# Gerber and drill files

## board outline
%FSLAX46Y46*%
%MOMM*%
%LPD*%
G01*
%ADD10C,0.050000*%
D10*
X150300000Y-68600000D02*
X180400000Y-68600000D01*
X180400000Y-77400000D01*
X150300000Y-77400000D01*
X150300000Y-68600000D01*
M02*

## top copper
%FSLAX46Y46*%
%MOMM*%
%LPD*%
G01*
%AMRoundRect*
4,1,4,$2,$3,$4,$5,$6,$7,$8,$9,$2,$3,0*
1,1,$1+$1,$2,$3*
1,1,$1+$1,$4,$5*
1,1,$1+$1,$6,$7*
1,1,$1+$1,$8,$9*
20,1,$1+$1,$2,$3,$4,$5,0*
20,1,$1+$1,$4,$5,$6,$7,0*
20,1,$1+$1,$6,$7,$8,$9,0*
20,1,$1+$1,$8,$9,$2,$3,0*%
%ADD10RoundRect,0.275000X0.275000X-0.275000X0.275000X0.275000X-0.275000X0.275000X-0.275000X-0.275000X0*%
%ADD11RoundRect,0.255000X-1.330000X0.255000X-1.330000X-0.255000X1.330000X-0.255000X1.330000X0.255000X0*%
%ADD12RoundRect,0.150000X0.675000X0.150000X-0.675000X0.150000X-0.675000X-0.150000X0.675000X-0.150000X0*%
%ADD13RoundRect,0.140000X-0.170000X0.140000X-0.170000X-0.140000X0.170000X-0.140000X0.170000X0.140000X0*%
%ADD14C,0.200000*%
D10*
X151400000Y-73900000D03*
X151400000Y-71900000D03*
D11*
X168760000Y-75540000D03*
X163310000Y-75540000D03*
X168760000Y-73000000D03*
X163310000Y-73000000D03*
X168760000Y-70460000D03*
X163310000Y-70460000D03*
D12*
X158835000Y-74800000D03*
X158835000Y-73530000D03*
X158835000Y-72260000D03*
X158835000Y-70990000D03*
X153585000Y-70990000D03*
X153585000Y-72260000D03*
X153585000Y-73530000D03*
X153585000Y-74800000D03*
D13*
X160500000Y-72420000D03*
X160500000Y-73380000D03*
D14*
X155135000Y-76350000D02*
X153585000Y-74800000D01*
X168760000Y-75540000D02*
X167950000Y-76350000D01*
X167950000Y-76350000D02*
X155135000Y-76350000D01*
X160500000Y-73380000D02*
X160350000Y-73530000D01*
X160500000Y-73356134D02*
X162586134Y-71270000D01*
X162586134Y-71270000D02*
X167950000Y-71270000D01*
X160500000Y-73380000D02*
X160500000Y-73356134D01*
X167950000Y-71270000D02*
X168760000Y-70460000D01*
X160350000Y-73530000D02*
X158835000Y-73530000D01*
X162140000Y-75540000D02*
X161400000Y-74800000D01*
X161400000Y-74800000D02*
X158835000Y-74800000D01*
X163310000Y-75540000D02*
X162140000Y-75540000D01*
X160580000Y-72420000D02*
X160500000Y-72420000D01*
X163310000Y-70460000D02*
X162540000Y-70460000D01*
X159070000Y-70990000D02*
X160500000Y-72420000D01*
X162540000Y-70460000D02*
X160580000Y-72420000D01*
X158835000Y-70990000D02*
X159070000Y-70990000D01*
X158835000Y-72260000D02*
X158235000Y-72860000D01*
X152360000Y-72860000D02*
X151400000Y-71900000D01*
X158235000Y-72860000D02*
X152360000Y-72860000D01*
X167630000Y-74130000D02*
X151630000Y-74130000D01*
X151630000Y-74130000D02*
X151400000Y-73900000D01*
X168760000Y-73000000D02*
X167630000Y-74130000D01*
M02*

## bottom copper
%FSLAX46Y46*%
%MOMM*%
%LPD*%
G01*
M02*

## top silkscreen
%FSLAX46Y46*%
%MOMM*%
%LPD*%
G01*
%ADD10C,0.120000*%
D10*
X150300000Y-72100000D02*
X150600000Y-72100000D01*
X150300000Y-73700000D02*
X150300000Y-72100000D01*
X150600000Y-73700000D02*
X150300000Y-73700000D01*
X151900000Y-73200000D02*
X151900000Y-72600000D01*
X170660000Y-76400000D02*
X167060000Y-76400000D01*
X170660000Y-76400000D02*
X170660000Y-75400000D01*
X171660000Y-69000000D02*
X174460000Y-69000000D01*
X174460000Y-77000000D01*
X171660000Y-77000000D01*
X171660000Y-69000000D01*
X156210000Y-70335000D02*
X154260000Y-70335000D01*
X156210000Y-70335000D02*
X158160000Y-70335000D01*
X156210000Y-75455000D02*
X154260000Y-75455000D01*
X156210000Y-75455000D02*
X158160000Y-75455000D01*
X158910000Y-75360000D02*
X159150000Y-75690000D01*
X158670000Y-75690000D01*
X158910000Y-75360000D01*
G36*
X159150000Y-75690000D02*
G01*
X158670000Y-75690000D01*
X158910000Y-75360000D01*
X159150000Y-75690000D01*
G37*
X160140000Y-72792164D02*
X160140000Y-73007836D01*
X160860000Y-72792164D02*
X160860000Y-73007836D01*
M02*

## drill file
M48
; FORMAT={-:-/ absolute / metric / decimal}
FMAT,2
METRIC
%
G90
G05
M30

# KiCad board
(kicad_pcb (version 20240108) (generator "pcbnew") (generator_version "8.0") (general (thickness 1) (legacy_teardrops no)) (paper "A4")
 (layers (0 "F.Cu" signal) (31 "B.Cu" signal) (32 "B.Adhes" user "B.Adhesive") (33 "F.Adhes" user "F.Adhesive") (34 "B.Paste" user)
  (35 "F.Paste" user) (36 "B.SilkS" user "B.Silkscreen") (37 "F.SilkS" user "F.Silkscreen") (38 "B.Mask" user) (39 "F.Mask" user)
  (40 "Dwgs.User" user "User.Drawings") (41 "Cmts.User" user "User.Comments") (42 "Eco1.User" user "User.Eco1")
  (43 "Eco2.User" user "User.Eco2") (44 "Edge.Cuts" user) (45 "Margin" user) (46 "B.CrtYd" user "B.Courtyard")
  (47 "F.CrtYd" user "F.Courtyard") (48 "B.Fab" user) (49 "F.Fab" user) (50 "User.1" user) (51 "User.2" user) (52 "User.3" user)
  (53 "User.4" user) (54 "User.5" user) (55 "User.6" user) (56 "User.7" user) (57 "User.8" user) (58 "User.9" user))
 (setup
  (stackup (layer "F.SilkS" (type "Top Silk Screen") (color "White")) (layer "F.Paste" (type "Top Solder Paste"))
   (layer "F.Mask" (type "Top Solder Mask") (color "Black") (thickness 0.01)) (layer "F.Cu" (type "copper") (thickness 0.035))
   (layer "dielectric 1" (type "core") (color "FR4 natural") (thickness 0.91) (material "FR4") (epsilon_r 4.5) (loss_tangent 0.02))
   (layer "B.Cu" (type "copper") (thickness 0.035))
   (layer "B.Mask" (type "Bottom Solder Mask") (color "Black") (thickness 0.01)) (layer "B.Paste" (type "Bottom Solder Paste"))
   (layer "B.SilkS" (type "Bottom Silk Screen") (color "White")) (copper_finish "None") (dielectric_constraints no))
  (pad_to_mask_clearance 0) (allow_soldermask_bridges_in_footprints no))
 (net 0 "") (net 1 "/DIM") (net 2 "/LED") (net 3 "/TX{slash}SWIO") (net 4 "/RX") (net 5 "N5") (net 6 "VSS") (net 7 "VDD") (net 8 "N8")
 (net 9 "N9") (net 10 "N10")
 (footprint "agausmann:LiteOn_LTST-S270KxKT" (layer "F.Cu") (at 151.4 72.9 90)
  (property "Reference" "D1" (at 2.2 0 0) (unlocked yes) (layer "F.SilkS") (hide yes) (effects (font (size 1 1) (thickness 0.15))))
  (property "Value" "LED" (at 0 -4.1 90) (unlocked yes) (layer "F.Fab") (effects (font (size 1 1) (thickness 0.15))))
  (fp_line (start 0.8 -1.1) (end 0.8 -0.8) (stroke (width 0.12) (type default)) (layer "F.SilkS"))
  (fp_line (start -0.8 -1.1) (end 0.8 -1.1) (stroke (width 0.12) (type default)) (layer "F.SilkS"))
  (fp_line (start -0.8 -0.8) (end -0.8 -1.1) (stroke (width 0.12) (type default)) (layer "F.SilkS"))
  (fp_line (start -0.3 0.5) (end 0.3 0.5) (stroke (width 0.12) (type default)) (layer "F.SilkS"))
  (pad "1" smd roundrect (at -1 0 90) (size 1.1 1.1) (layers "F.Cu" "F.Paste" "F.Mask") (roundrect_rratio 0.25) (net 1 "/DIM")
   (thermal_bridge_angle 45))
  (pad "2" smd roundrect (at 1 0 90) (size 1.1 1.1) (layers "F.Cu" "F.Paste" "F.Mask") (roundrect_rratio 0.25) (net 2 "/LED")
   (thermal_bridge_angle 45)))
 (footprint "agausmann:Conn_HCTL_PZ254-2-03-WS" (layer "F.Cu") (at 173.06 73 90)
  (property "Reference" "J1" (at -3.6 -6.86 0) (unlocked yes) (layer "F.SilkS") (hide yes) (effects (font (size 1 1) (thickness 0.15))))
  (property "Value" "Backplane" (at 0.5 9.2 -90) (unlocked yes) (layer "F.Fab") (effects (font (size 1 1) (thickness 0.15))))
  (fp_line (start -3.4 -2.4) (end -3.4 -6) (stroke (width 0.12) (type default)) (layer "F.SilkS"))
  (fp_line (start -3.4 -2.4) (end -2.4 -2.4) (stroke (width 0.12) (type default)) (layer "F.SilkS"))
  (fp_rect (start -4 -1.4) (end 4 1.4) (stroke (width 0.12) (type default)) (fill none) (layer "F.SilkS"))
  (pad "1" smd roundrect (at -2.54 -4.3 270) (size 1.02 3.17) (layers "F.Cu" "F.Paste" "F.Mask") (roundrect_rratio 0.25)
   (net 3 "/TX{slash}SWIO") (thermal_bridge_angle 45))
  (pad "2" smd roundrect (at -2.54 -9.75 270) (size 1.02 3.17) (layers "F.Cu" "F.Paste" "F.Mask") (roundrect_rratio 0.25) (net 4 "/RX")
   (thermal_bridge_angle 45))
  (pad "3" smd roundrect (at 0 -4.3 270) (size 1.02 3.17) (layers "F.Cu" "F.Paste" "F.Mask") (roundrect_rratio 0.25) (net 1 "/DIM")
   (thermal_bridge_angle 45))
  (pad "4" smd roundrect (at 0 -9.75 270) (size 1.02 3.17) (layers "F.Cu" "F.Paste" "F.Mask") (roundrect_rratio 0.25) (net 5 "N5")
   (thermal_bridge_angle 45))
  (pad "5" smd roundrect (at 2.54 -4.3 270) (size 1.02 3.17) (layers "F.Cu" "F.Paste" "F.Mask") (roundrect_rratio 0.25) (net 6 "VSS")
   (thermal_bridge_angle 45))
  (pad "6" smd roundrect (at 2.54 -9.75 270) (size 1.02 3.17) (layers "F.Cu" "F.Paste" "F.Mask") (roundrect_rratio 0.25) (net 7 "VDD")
   (thermal_bridge_angle 45)))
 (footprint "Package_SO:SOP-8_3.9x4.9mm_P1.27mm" (layer "F.Cu") (at 156.21 72.895 180)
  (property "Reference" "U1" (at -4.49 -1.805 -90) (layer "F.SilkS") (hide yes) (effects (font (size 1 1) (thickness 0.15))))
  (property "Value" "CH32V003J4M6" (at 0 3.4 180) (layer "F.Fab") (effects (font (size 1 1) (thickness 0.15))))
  (fp_line (start 0 2.56) (end 1.95 2.56) (stroke (width 0.12) (type solid)) (layer "F.SilkS"))
  (fp_line (start 0 2.56) (end -1.95 2.56) (stroke (width 0.12) (type solid)) (layer "F.SilkS"))
  (fp_line (start 0 -2.56) (end 1.95 -2.56) (stroke (width 0.12) (type solid)) (layer "F.SilkS"))
  (fp_line (start 0 -2.56) (end -1.95 -2.56) (stroke (width 0.12) (type solid)) (layer "F.SilkS"))
  (fp_poly
   (pts (xy -2.7 -2.465) (xy -2.94 -2.795) (xy -2.46 -2.795) (xy -2.7 -2.465)) (stroke (width 0.12) (type solid)) (fill solid)
   (layer "F.SilkS"))
  (pad "1" smd roundrect (at -2.625 -1.905 180) (size 1.65 0.6) (layers "F.Cu" "F.Paste" "F.Mask") (roundrect_rratio 0.25) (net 4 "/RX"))
  (pad "2" smd roundrect (at -2.625 -0.635 180) (size 1.65 0.6) (layers "F.Cu" "F.Paste" "F.Mask") (roundrect_rratio 0.25) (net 6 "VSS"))
  (pad "3" smd roundrect (at -2.625 0.635 180) (size 1.65 0.6) (layers "F.Cu" "F.Paste" "F.Mask") (roundrect_rratio 0.25) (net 2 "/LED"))
  (pad "4" smd roundrect (at -2.625 1.905 180) (size 1.65 0.6) (layers "F.Cu" "F.Paste" "F.Mask") (roundrect_rratio 0.25) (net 7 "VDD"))
  (pad "5" smd roundrect (at 2.625 1.905 180) (size 1.65 0.6) (layers "F.Cu" "F.Paste" "F.Mask") (roundrect_rratio 0.25) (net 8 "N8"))
  (pad "6" smd roundrect (at 2.625 0.635 180) (size 1.65 0.6) (layers "F.Cu" "F.Paste" "F.Mask") (roundrect_rratio 0.25) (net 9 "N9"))
  (pad "7" smd roundrect (at 2.625 -0.635 180) (size 1.65 0.6) (layers "F.Cu" "F.Paste" "F.Mask") (roundrect_rratio 0.25) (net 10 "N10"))
  (pad "8" smd roundrect (at 2.625 -1.905 180) (size 1.65 0.6) (layers "F.Cu" "F.Paste" "F.Mask") (roundrect_rratio 0.25)
   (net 3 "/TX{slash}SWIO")))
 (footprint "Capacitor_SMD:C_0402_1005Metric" (layer "F.Cu") (at 160.5 72.9 -90)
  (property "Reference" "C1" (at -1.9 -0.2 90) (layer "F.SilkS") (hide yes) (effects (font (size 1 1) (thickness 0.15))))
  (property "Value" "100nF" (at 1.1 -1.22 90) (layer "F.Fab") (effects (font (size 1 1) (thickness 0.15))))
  (fp_line (start -0.107836 0.36) (end 0.107836 0.36) (stroke (width 0.12) (type solid)) (layer "F.SilkS"))
  (fp_line (start -0.107836 -0.36) (end 0.107836 -0.36) (stroke (width 0.12) (type solid)) (layer "F.SilkS"))
  (pad "1" smd roundrect (at -0.48 0 270) (size 0.56 0.62) (layers "F.Cu" "F.Paste" "F.Mask") (roundrect_rratio 0.25) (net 7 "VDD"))
  (pad "2" smd roundrect (at 0.48 0 270) (size 0.56 0.62) (layers "F.Cu" "F.Paste" "F.Mask") (roundrect_rratio 0.25) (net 6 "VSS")))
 (gr_rect (start 150.3 68.6) (end 180.4 77.4) (stroke (width 0.05) (type default)) (fill none) (layer "Edge.Cuts"))
 (segment (start 155.135 76.35) (end 153.585 74.8) (width 0.2) (layer "F.Cu") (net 3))
 (segment (start 168.76 75.54) (end 167.95 76.35) (width 0.2) (layer "F.Cu") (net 3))
 (segment (start 167.95 76.35) (end 155.135 76.35) (width 0.2) (layer "F.Cu") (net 3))
 (segment (start 160.5 73.38) (end 160.35 73.53) (width 0.2) (layer "F.Cu") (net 6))
 (segment (start 160.5 73.356134) (end 162.586134 71.27) (width 0.2) (layer "F.Cu") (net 6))
 (segment (start 162.586134 71.27) (end 167.95 71.27) (width 0.2) (layer "F.Cu") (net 6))
 (segment (start 160.5 73.38) (end 160.5 73.356134) (width 0.2) (layer "F.Cu") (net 6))
 (segment (start 167.95 71.27) (end 168.76 70.46) (width 0.2) (layer "F.Cu") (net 6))
 (segment (start 160.35 73.53) (end 158.835 73.53) (width 0.2) (layer "F.Cu") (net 6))
 (segment (start 162.14 75.54) (end 161.4 74.8) (width 0.2) (layer "F.Cu") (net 4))
 (segment (start 161.4 74.8) (end 158.835 74.8) (width 0.2) (layer "F.Cu") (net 4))
 (segment (start 163.31 75.54) (end 162.14 75.54) (width 0.2) (layer "F.Cu") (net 4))
 (segment (start 160.58 72.42) (end 160.5 72.42) (width 0.2) (layer "F.Cu") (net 7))
 (segment (start 163.31 70.46) (end 162.54 70.46) (width 0.2) (layer "F.Cu") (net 7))
 (segment (start 159.07 70.99) (end 160.5 72.42) (width 0.2) (layer "F.Cu") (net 7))
 (segment (start 162.54 70.46) (end 160.58 72.42) (width 0.2) (layer "F.Cu") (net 7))
 (segment (start 158.835 70.99) (end 159.07 70.99) (width 0.2) (layer "F.Cu") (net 7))
 (segment (start 158.835 72.26) (end 158.235 72.86) (width 0.2) (layer "F.Cu") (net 2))
 (segment (start 152.36 72.86) (end 151.4 71.9) (width 0.2) (layer "F.Cu") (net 2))
 (segment (start 158.235 72.86) (end 152.36 72.86) (width 0.2) (layer "F.Cu") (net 2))
 (segment (start 167.63 74.13) (end 151.63 74.13) (width 0.2) (layer "F.Cu") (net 1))
 (segment (start 151.63 74.13) (end 151.4 73.9) (width 0.2) (layer "F.Cu") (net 1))
 (segment (start 168.76 73) (end 167.63 74.13) (width 0.2) (layer "F.Cu") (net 1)))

